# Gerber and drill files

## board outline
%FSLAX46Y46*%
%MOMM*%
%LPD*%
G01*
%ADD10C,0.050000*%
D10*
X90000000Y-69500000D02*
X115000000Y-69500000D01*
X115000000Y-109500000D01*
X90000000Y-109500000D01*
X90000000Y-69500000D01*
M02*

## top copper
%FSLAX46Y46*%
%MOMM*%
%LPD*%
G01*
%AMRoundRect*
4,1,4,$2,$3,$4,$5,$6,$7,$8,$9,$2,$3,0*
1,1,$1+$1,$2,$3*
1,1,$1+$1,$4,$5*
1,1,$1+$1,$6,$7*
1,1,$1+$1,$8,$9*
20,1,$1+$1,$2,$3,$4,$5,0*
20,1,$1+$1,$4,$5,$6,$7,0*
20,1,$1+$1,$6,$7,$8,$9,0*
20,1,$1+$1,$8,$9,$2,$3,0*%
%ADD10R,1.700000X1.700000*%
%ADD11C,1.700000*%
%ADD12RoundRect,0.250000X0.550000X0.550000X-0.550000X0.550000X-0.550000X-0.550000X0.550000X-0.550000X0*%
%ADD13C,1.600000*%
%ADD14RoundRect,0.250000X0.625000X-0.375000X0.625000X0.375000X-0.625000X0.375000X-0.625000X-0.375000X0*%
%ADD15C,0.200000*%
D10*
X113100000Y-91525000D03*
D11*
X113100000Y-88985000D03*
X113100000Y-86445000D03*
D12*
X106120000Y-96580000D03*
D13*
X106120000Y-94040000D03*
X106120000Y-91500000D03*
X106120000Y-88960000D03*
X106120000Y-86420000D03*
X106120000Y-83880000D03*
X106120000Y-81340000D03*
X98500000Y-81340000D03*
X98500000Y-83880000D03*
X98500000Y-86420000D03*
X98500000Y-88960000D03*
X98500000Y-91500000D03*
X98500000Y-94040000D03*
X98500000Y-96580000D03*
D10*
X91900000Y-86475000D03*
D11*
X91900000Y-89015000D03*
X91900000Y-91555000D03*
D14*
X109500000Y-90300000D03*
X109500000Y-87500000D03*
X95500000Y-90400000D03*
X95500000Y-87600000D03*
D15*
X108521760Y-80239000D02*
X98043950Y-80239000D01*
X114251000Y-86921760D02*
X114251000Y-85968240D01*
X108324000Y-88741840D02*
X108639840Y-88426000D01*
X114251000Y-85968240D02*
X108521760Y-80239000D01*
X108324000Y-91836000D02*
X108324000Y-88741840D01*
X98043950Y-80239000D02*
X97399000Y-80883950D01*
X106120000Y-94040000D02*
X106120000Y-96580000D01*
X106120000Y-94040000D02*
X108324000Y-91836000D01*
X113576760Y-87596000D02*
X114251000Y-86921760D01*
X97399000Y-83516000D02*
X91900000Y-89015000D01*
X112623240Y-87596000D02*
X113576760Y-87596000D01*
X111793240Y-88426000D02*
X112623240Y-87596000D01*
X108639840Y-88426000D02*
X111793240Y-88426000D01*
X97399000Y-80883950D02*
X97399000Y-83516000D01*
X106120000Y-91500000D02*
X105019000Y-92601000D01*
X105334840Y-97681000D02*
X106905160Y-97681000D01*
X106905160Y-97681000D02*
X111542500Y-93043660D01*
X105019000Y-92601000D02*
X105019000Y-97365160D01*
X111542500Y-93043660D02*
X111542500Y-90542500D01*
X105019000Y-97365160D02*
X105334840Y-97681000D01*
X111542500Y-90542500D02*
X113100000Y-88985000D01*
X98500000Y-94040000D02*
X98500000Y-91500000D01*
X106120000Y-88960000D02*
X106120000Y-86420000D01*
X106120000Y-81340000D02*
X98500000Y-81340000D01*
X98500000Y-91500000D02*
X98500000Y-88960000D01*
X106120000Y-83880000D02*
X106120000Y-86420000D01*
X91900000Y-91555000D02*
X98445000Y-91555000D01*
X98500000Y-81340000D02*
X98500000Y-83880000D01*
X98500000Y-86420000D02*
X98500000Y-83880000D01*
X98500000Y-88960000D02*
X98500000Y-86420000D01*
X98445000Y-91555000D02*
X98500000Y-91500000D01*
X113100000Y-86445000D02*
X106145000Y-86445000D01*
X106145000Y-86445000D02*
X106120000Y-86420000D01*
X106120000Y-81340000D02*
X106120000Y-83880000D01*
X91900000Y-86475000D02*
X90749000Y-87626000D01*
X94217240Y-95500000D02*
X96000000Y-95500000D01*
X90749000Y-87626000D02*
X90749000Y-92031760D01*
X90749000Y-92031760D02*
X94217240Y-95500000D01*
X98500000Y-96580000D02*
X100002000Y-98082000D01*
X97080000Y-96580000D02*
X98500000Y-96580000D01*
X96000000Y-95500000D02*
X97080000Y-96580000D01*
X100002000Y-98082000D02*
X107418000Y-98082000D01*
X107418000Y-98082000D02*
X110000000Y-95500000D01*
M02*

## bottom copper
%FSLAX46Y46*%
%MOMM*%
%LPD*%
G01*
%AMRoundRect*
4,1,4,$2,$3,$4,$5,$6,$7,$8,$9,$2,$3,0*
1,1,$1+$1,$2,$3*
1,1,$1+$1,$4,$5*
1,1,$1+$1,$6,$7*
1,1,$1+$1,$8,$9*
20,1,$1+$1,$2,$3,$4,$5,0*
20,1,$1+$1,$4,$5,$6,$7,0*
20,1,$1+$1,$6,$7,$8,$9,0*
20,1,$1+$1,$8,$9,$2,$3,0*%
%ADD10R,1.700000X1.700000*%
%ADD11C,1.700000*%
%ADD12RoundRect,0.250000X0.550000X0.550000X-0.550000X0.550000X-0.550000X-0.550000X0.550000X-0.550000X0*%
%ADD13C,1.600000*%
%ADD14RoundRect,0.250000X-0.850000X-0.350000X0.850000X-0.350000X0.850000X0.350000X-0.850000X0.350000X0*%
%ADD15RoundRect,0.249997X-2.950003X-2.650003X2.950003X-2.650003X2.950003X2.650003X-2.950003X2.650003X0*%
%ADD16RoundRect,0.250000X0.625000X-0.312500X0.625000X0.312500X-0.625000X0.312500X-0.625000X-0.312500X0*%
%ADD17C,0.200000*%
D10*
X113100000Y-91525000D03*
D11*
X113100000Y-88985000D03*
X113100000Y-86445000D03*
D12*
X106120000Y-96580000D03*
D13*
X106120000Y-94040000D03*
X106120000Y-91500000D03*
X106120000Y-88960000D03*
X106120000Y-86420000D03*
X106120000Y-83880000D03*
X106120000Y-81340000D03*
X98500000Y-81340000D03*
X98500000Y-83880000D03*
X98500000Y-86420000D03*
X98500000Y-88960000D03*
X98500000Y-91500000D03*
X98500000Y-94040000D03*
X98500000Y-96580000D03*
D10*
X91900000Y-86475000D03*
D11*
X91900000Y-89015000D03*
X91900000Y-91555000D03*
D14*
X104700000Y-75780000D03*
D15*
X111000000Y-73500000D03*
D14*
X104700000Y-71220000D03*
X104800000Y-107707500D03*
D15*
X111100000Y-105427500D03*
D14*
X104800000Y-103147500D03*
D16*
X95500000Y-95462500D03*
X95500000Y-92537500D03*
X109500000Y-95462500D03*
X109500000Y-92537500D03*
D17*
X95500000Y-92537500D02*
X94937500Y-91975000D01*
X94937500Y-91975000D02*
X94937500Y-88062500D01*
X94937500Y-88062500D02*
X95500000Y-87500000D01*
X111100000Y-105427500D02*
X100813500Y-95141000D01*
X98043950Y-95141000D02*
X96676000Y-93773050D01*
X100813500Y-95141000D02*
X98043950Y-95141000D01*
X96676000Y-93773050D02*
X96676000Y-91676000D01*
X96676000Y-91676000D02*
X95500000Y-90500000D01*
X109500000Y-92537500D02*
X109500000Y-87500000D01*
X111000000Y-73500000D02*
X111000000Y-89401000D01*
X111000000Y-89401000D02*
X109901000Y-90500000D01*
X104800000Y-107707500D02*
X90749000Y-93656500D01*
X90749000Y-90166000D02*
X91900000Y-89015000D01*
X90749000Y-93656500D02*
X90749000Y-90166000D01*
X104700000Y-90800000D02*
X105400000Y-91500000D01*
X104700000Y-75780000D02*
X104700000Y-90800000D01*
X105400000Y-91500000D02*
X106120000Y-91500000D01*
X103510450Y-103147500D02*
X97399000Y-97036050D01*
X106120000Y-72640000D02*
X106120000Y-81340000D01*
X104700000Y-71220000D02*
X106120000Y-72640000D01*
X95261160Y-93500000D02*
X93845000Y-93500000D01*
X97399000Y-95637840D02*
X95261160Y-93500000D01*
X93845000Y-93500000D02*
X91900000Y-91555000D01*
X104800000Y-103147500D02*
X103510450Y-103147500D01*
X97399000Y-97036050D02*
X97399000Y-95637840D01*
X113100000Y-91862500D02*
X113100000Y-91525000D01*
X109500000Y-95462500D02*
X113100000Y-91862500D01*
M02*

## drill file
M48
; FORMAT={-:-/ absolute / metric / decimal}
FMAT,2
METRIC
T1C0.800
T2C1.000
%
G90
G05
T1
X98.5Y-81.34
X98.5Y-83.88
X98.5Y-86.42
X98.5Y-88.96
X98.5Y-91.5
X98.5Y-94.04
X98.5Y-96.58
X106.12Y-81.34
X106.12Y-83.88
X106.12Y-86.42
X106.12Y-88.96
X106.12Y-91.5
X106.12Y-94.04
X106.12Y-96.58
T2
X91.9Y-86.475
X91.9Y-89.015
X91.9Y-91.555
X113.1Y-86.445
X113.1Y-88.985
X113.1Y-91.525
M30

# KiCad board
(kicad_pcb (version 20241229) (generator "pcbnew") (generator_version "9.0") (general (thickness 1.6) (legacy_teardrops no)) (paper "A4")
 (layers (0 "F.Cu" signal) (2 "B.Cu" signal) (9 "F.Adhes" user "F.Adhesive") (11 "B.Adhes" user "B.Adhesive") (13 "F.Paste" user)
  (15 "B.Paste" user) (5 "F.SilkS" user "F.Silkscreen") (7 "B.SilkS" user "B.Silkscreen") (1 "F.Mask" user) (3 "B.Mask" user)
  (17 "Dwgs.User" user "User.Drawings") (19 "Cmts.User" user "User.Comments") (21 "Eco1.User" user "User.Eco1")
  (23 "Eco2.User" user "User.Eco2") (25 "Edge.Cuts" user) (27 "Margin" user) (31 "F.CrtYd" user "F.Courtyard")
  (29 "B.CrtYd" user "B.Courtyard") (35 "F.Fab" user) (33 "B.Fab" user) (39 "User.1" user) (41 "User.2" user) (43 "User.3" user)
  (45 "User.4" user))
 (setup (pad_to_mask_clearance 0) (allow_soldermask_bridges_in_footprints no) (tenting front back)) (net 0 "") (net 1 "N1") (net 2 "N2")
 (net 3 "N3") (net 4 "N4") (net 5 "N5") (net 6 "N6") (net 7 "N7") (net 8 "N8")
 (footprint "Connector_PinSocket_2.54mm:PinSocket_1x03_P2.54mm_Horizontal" (layer "F.Cu") (at 113.1 91.525 180)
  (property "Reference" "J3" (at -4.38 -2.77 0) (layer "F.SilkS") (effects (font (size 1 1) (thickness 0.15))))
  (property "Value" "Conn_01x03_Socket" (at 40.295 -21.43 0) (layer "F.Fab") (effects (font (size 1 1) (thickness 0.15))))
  (pad "1" thru_hole rect (at 0 0 180) (size 1.7 1.7) (drill 1) (layers "*.Cu" "*.Mask") (remove_unused_layers no) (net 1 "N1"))
  (pad "2" thru_hole circle (at 0 2.54 180) (size 1.7 1.7) (drill 1) (layers "*.Cu" "*.Mask") (remove_unused_layers no) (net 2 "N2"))
  (pad "3" thru_hole circle (at 0 5.08 180) (size 1.7 1.7) (drill 1) (layers "*.Cu" "*.Mask") (remove_unused_layers no) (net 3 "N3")))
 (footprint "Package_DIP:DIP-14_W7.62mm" (layer "F.Cu") (at 106.12 96.58 180)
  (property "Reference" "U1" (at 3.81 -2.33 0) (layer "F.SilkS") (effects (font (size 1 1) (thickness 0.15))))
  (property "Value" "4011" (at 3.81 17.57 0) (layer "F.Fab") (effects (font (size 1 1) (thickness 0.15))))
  (pad "1" thru_hole roundrect (at 0 0 180) (size 1.6 1.6) (drill 0.8) (layers "*.Cu" "*.Mask") (remove_unused_layers no)
   (roundrect_rratio 0.15625) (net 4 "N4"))
  (pad "2" thru_hole circle (at 0 2.54 180) (size 1.6 1.6) (drill 0.8) (layers "*.Cu" "*.Mask") (remove_unused_layers no) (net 4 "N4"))
  (pad "3" thru_hole circle (at 0 5.08 180) (size 1.6 1.6) (drill 0.8) (layers "*.Cu" "*.Mask") (remove_unused_layers no) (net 2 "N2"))
  (pad "4" thru_hole circle (at 0 7.62 180) (size 1.6 1.6) (drill 0.8) (layers "*.Cu" "*.Mask") (remove_unused_layers no) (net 3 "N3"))
  (pad "5" thru_hole circle (at 0 10.16 180) (size 1.6 1.6) (drill 0.8) (layers "*.Cu" "*.Mask") (remove_unused_layers no) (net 3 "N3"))
  (pad "6" thru_hole circle (at 0 12.7 180) (size 1.6 1.6) (drill 0.8) (layers "*.Cu" "*.Mask") (remove_unused_layers no) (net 3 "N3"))
  (pad "7" thru_hole circle (at 0 15.24 180) (size 1.6 1.6) (drill 0.8) (layers "*.Cu" "*.Mask") (remove_unused_layers no) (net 3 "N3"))
  (pad "8" thru_hole circle (at 7.62 15.24 180) (size 1.6 1.6) (drill 0.8) (layers "*.Cu" "*.Mask") (remove_unused_layers no) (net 3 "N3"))
  (pad "9" thru_hole circle (at 7.62 12.7 180) (size 1.6 1.6) (drill 0.8) (layers "*.Cu" "*.Mask") (remove_unused_layers no) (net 3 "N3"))
  (pad "10" thru_hole circle (at 7.62 10.16 180) (size 1.6 1.6) (drill 0.8) (layers "*.Cu" "*.Mask") (remove_unused_layers no) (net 3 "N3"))
  (pad "11" thru_hole circle (at 7.62 7.62 180) (size 1.6 1.6) (drill 0.8) (layers "*.Cu" "*.Mask") (remove_unused_layers no) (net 3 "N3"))
  (pad "12" thru_hole circle (at 7.62 5.08 180) (size 1.6 1.6) (drill 0.8) (layers "*.Cu" "*.Mask") (remove_unused_layers no) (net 3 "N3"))
  (pad "13" thru_hole circle (at 7.62 2.54 180) (size 1.6 1.6) (drill 0.8) (layers "*.Cu" "*.Mask") (remove_unused_layers no) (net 3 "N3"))
  (pad "14" thru_hole circle (at 7.62 0 180) (size 1.6 1.6) (drill 0.8) (layers "*.Cu" "*.Mask") (remove_unused_layers no) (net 1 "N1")))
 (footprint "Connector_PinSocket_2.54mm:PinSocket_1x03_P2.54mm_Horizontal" (layer "F.Cu") (at 91.9 86.475)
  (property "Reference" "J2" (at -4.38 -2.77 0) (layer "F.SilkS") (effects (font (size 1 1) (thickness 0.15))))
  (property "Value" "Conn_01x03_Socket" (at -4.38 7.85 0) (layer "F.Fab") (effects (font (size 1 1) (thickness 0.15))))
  (pad "1" thru_hole rect (at 0 0) (size 1.7 1.7) (drill 1) (layers "*.Cu" "*.Mask") (remove_unused_layers no) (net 1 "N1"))
  (pad "2" thru_hole circle (at 0 2.54) (size 1.7 1.7) (drill 1) (layers "*.Cu" "*.Mask") (remove_unused_layers no) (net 4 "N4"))
  (pad "3" thru_hole circle (at 0 5.08) (size 1.7 1.7) (drill 1) (layers "*.Cu" "*.Mask") (remove_unused_layers no) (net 3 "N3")))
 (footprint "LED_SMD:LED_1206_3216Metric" (layer "F.Cu") (at 109.5 88.9 90)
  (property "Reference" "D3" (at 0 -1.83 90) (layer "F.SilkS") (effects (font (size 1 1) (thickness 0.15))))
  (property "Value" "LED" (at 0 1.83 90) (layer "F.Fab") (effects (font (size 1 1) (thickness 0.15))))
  (pad "1" smd roundrect (at -1.4 0 90) (size 1.25 1.75) (layers "F.Cu" "F.Mask" "F.Paste") (roundrect_rratio 0.2) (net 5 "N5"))
  (pad "2" smd roundrect (at 1.4 0 90) (size 1.25 1.75) (layers "F.Cu" "F.Mask" "F.Paste") (roundrect_rratio 0.2) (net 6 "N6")))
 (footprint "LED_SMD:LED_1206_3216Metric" (layer "F.Cu") (at 95.5 89 90)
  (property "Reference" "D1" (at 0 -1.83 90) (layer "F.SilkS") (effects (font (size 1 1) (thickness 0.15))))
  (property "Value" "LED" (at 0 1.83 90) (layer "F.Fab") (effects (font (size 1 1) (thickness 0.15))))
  (pad "1" smd roundrect (at -1.4 0 90) (size 1.25 1.75) (layers "F.Cu" "F.Mask" "F.Paste") (roundrect_rratio 0.2) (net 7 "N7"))
  (pad "2" smd roundrect (at 1.4 0 90) (size 1.25 1.75) (layers "F.Cu" "F.Mask" "F.Paste") (roundrect_rratio 0.2) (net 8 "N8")))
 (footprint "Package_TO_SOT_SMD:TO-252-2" (layer "B.Cu") (at 109.74 73.5)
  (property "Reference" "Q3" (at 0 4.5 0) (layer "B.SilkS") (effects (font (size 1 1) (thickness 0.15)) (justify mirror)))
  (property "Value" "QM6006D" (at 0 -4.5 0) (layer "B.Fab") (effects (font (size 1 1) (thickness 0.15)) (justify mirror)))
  (pad "" smd roundrect (at -0.415 -1.525) (size 3.05 2.75) (layers "B.Paste") (roundrect_rratio 0.090909))
  (pad "" smd roundrect (at -0.415 1.525) (size 3.05 2.75) (layers "B.Paste") (roundrect_rratio 0.090909))
  (pad "" smd roundrect (at 2.935 -1.525) (size 3.05 2.75) (layers "B.Paste") (roundrect_rratio 0.090909))
  (pad "" smd roundrect (at 2.935 1.525) (size 3.05 2.75) (layers "B.Paste") (roundrect_rratio 0.090909))
  (pad "1" smd roundrect (at -5.04 2.28) (size 2.2 1.2) (layers "B.Cu" "B.Mask" "B.Paste") (roundrect_rratio 0.208333) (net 2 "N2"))
  (pad "2" smd roundrect (at 1.26 0) (size 6.4 5.8) (layers "B.Cu" "B.Mask") (roundrect_rratio 0.043103) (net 5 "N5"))
  (pad "3" smd roundrect (at -5.04 -2.28) (size 2.2 1.2) (layers "B.Cu" "B.Mask" "B.Paste") (roundrect_rratio 0.208333) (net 3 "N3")))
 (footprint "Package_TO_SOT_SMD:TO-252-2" (layer "B.Cu") (at 109.84 105.4275)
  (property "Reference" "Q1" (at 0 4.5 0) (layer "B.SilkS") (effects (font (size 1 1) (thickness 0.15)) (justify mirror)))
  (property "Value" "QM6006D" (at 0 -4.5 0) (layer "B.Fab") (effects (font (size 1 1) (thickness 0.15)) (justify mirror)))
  (pad "" smd roundrect (at -0.415 -1.525) (size 3.05 2.75) (layers "B.Paste") (roundrect_rratio 0.090909))
  (pad "" smd roundrect (at -0.415 1.525) (size 3.05 2.75) (layers "B.Paste") (roundrect_rratio 0.090909))
  (pad "" smd roundrect (at 2.935 -1.525) (size 3.05 2.75) (layers "B.Paste") (roundrect_rratio 0.090909))
  (pad "" smd roundrect (at 2.935 1.525) (size 3.05 2.75) (layers "B.Paste") (roundrect_rratio 0.090909))
  (pad "1" smd roundrect (at -5.04 2.28) (size 2.2 1.2) (layers "B.Cu" "B.Mask" "B.Paste") (roundrect_rratio 0.208333) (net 4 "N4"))
  (pad "2" smd roundrect (at 1.26 0) (size 6.4 5.8) (layers "B.Cu" "B.Mask") (roundrect_rratio 0.043103) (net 7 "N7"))
  (pad "3" smd roundrect (at -5.04 -2.28) (size 2.2 1.2) (layers "B.Cu" "B.Mask" "B.Paste") (roundrect_rratio 0.208333) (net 3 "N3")))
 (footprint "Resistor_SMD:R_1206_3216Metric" (layer "B.Cu") (at 95.5 94 90)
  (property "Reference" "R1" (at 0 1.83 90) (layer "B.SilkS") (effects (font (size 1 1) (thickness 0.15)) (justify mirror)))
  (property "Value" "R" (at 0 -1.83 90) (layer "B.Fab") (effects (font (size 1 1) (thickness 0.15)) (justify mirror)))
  (pad "1" smd roundrect (at -1.4625 0 90) (size 1.125 1.75) (layers "B.Cu" "B.Mask" "B.Paste") (roundrect_rratio 0.222222) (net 1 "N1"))
  (pad "2" smd roundrect (at 1.4625 0 90) (size 1.125 1.75) (layers "B.Cu" "B.Mask" "B.Paste") (roundrect_rratio 0.222222) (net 8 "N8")))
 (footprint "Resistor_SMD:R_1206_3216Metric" (layer "B.Cu") (at 109.5 94 90)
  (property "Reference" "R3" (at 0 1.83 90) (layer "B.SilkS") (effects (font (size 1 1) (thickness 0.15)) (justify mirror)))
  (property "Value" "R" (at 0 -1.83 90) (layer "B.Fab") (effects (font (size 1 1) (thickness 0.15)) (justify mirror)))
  (pad "1" smd roundrect (at -1.4625 0 90) (size 1.125 1.75) (layers "B.Cu" "B.Mask" "B.Paste") (roundrect_rratio 0.222222) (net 1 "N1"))
  (pad "2" smd roundrect (at 1.4625 0 90) (size 1.125 1.75) (layers "B.Cu" "B.Mask" "B.Paste") (roundrect_rratio 0.222222) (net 6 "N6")))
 (gr_rect (start 90 69.5) (end 115 109.5) (stroke (width 0.05) (type default)) (fill no) (layer "Edge.Cuts"))
 (segment (start 95.5 92.5375) (end 94.9375 91.975) (width 0.2) (layer "B.Cu") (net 8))
 (segment (start 94.9375 91.975) (end 94.9375 88.0625) (width 0.2) (layer "B.Cu") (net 8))
 (segment (start 94.9375 88.0625) (end 95.5 87.5) (width 0.2) (layer "B.Cu") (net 8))
 (segment (start 111.1 105.4275) (end 100.8135 95.141) (width 0.2) (layer "B.Cu") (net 7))
 (segment (start 98.04395 95.141) (end 96.676 93.77305) (width 0.2) (layer "B.Cu") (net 7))
 (segment (start 100.8135 95.141) (end 98.04395 95.141) (width 0.2) (layer "B.Cu") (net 7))
 (segment (start 96.676 93.77305) (end 96.676 91.676) (width 0.2) (layer "B.Cu") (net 7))
 (segment (start 96.676 91.676) (end 95.5 90.5) (width 0.2) (layer "B.Cu") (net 7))
 (segment (start 109.5 92.5375) (end 109.5 87.5) (width 0.2) (layer "B.Cu") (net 6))
 (segment (start 111 73.5) (end 111 89.401) (width 0.2) (layer "B.Cu") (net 5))
 (segment (start 111 89.401) (end 109.901 90.5) (width 0.2) (layer "B.Cu") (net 5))
 (segment (start 108.52176 80.239) (end 98.04395 80.239) (width 0.2) (layer "F.Cu") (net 4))
 (segment (start 114.251 86.92176) (end 114.251 85.96824) (width 0.2) (layer "F.Cu") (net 4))
 (segment (start 108.324 88.74184) (end 108.63984 88.426) (width 0.2) (layer "F.Cu") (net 4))
 (segment (start 114.251 85.96824) (end 108.52176 80.239) (width 0.2) (layer "F.Cu") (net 4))
 (segment (start 108.324 91.836) (end 108.324 88.74184) (width 0.2) (layer "F.Cu") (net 4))
 (segment (start 98.04395 80.239) (end 97.399 80.88395) (width 0.2) (layer "F.Cu") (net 4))
 (segment (start 106.12 94.04) (end 106.12 96.58) (width 0.2) (layer "F.Cu") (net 4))
 (segment (start 106.12 94.04) (end 108.324 91.836) (width 0.2) (layer "F.Cu") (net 4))
 (segment (start 113.57676 87.596) (end 114.251 86.92176) (width 0.2) (layer "F.Cu") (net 4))
 (segment (start 97.399 83.516) (end 91.9 89.015) (width 0.2) (layer "F.Cu") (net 4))
 (segment (start 112.62324 87.596) (end 113.57676 87.596) (width 0.2) (layer "F.Cu") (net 4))
 (segment (start 111.79324 88.426) (end 112.62324 87.596) (width 0.2) (layer "F.Cu") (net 4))
 (segment (start 108.63984 88.426) (end 111.79324 88.426) (width 0.2) (layer "F.Cu") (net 4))
 (segment (start 97.399 80.88395) (end 97.399 83.516) (width 0.2) (layer "F.Cu") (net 4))
 (segment (start 104.8 107.7075) (end 90.749 93.6565) (width 0.2) (layer "B.Cu") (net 4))
 (segment (start 90.749 90.166) (end 91.9 89.015) (width 0.2) (layer "B.Cu") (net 4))
 (segment (start 90.749 93.6565) (end 90.749 90.166) (width 0.2) (layer "B.Cu") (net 4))
 (segment (start 106.12 91.5) (end 105.019 92.601) (width 0.2) (layer "F.Cu") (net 2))
 (segment (start 105.33484 97.681) (end 106.90516 97.681) (width 0.2) (layer "F.Cu") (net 2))
 (segment (start 106.90516 97.681) (end 111.5425 93.04366) (width 0.2) (layer "F.Cu") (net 2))
 (segment (start 105.019 92.601) (end 105.019 97.36516) (width 0.2) (layer "F.Cu") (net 2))
 (segment (start 111.5425 93.04366) (end 111.5425 90.5425) (width 0.2) (layer "F.Cu") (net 2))
 (segment (start 105.019 97.36516) (end 105.33484 97.681) (width 0.2) (layer "F.Cu") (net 2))
 (segment (start 111.5425 90.5425) (end 113.1 88.985) (width 0.2) (layer "F.Cu") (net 2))
 (segment (start 104.7 90.8) (end 105.4 91.5) (width 0.2) (layer "B.Cu") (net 2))
 (segment (start 104.7 75.78) (end 104.7 90.8) (width 0.2) (layer "B.Cu") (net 2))
 (segment (start 105.4 91.5) (end 106.12 91.5) (width 0.2) (layer "B.Cu") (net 2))
 (segment (start 98.5 94.04) (end 98.5 91.5) (width 0.2) (layer "F.Cu") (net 3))
 (segment (start 106.12 88.96) (end 106.12 86.42) (width 0.2) (layer "F.Cu") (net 3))
 (segment (start 106.12 81.34) (end 98.5 81.34) (width 0.2) (layer "F.Cu") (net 3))
 (segment (start 98.5 91.5) (end 98.5 88.96) (width 0.2) (layer "F.Cu") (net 3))
 (segment (start 106.12 83.88) (end 106.12 86.42) (width 0.2) (layer "F.Cu") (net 3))
 (segment (start 91.9 91.555) (end 98.445 91.555) (width 0.2) (layer "F.Cu") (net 3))
 (segment (start 98.5 81.34) (end 98.5 83.88) (width 0.2) (layer "F.Cu") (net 3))
 (segment (start 98.5 86.42) (end 98.5 83.88) (width 0.2) (layer "F.Cu") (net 3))
 (segment (start 98.5 88.96) (end 98.5 86.42) (width 0.2) (layer "F.Cu") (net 3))
 (segment (start 98.445 91.555) (end 98.5 91.5) (width 0.2) (layer "F.Cu") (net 3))
 (segment (start 113.1 86.445) (end 106.145 86.445) (width 0.2) (layer "F.Cu") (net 3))
 (segment (start 106.145 86.445) (end 106.12 86.42) (width 0.2) (layer "F.Cu") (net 3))
 (segment (start 106.12 81.34) (end 106.12 83.88) (width 0.2) (layer "F.Cu") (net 3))
 (segment (start 103.51045 103.1475) (end 97.399 97.03605) (width 0.2) (layer "B.Cu") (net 3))
 (segment (start 106.12 72.64) (end 106.12 81.34) (width 0.2) (layer "B.Cu") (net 3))
 (segment (start 104.7 71.22) (end 106.12 72.64) (width 0.2) (layer "B.Cu") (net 3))
 (segment (start 95.26116 93.5) (end 93.845 93.5) (width 0.2) (layer "B.Cu") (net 3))
 (segment (start 97.399 95.63784) (end 95.26116 93.5) (width 0.2) (layer "B.Cu") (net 3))
 (segment (start 93.845 93.5) (end 91.9 91.555) (width 0.2) (layer "B.Cu") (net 3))
 (segment (start 104.8 103.1475) (end 103.51045 103.1475) (width 0.2) (layer "B.Cu") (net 3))
 (segment (start 97.399 97.03605) (end 97.399 95.63784) (width 0.2) (layer "B.Cu") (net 3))
 (segment (start 91.9 86.475) (end 90.749 87.626) (width 0.2) (layer "F.Cu") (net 1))
 (segment (start 94.21724 95.5) (end 96 95.5) (width 0.2) (layer "F.Cu") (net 1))
 (segment (start 90.749 87.626) (end 90.749 92.03176) (width 0.2) (layer "F.Cu") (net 1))
 (segment (start 90.749 92.03176) (end 94.21724 95.5) (width 0.2) (layer "F.Cu") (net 1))
 (segment (start 98.5 96.58) (end 100.002 98.082) (width 0.2) (layer "F.Cu") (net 1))
 (segment (start 97.08 96.58) (end 98.5 96.58) (width 0.2) (layer "F.Cu") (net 1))
 (segment (start 96 95.5) (end 97.08 96.58) (width 0.2) (layer "F.Cu") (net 1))
 (segment (start 100.002 98.082) (end 107.418 98.082) (width 0.2) (layer "F.Cu") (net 1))
 (segment (start 107.418 98.082) (end 110 95.5) (width 0.2) (layer "F.Cu") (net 1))
 (segment (start 113.1 91.8625) (end 113.1 91.525) (width 0.2) (layer "B.Cu") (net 1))
 (segment (start 109.5 95.4625) (end 113.1 91.8625) (width 0.2) (layer "B.Cu") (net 1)))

